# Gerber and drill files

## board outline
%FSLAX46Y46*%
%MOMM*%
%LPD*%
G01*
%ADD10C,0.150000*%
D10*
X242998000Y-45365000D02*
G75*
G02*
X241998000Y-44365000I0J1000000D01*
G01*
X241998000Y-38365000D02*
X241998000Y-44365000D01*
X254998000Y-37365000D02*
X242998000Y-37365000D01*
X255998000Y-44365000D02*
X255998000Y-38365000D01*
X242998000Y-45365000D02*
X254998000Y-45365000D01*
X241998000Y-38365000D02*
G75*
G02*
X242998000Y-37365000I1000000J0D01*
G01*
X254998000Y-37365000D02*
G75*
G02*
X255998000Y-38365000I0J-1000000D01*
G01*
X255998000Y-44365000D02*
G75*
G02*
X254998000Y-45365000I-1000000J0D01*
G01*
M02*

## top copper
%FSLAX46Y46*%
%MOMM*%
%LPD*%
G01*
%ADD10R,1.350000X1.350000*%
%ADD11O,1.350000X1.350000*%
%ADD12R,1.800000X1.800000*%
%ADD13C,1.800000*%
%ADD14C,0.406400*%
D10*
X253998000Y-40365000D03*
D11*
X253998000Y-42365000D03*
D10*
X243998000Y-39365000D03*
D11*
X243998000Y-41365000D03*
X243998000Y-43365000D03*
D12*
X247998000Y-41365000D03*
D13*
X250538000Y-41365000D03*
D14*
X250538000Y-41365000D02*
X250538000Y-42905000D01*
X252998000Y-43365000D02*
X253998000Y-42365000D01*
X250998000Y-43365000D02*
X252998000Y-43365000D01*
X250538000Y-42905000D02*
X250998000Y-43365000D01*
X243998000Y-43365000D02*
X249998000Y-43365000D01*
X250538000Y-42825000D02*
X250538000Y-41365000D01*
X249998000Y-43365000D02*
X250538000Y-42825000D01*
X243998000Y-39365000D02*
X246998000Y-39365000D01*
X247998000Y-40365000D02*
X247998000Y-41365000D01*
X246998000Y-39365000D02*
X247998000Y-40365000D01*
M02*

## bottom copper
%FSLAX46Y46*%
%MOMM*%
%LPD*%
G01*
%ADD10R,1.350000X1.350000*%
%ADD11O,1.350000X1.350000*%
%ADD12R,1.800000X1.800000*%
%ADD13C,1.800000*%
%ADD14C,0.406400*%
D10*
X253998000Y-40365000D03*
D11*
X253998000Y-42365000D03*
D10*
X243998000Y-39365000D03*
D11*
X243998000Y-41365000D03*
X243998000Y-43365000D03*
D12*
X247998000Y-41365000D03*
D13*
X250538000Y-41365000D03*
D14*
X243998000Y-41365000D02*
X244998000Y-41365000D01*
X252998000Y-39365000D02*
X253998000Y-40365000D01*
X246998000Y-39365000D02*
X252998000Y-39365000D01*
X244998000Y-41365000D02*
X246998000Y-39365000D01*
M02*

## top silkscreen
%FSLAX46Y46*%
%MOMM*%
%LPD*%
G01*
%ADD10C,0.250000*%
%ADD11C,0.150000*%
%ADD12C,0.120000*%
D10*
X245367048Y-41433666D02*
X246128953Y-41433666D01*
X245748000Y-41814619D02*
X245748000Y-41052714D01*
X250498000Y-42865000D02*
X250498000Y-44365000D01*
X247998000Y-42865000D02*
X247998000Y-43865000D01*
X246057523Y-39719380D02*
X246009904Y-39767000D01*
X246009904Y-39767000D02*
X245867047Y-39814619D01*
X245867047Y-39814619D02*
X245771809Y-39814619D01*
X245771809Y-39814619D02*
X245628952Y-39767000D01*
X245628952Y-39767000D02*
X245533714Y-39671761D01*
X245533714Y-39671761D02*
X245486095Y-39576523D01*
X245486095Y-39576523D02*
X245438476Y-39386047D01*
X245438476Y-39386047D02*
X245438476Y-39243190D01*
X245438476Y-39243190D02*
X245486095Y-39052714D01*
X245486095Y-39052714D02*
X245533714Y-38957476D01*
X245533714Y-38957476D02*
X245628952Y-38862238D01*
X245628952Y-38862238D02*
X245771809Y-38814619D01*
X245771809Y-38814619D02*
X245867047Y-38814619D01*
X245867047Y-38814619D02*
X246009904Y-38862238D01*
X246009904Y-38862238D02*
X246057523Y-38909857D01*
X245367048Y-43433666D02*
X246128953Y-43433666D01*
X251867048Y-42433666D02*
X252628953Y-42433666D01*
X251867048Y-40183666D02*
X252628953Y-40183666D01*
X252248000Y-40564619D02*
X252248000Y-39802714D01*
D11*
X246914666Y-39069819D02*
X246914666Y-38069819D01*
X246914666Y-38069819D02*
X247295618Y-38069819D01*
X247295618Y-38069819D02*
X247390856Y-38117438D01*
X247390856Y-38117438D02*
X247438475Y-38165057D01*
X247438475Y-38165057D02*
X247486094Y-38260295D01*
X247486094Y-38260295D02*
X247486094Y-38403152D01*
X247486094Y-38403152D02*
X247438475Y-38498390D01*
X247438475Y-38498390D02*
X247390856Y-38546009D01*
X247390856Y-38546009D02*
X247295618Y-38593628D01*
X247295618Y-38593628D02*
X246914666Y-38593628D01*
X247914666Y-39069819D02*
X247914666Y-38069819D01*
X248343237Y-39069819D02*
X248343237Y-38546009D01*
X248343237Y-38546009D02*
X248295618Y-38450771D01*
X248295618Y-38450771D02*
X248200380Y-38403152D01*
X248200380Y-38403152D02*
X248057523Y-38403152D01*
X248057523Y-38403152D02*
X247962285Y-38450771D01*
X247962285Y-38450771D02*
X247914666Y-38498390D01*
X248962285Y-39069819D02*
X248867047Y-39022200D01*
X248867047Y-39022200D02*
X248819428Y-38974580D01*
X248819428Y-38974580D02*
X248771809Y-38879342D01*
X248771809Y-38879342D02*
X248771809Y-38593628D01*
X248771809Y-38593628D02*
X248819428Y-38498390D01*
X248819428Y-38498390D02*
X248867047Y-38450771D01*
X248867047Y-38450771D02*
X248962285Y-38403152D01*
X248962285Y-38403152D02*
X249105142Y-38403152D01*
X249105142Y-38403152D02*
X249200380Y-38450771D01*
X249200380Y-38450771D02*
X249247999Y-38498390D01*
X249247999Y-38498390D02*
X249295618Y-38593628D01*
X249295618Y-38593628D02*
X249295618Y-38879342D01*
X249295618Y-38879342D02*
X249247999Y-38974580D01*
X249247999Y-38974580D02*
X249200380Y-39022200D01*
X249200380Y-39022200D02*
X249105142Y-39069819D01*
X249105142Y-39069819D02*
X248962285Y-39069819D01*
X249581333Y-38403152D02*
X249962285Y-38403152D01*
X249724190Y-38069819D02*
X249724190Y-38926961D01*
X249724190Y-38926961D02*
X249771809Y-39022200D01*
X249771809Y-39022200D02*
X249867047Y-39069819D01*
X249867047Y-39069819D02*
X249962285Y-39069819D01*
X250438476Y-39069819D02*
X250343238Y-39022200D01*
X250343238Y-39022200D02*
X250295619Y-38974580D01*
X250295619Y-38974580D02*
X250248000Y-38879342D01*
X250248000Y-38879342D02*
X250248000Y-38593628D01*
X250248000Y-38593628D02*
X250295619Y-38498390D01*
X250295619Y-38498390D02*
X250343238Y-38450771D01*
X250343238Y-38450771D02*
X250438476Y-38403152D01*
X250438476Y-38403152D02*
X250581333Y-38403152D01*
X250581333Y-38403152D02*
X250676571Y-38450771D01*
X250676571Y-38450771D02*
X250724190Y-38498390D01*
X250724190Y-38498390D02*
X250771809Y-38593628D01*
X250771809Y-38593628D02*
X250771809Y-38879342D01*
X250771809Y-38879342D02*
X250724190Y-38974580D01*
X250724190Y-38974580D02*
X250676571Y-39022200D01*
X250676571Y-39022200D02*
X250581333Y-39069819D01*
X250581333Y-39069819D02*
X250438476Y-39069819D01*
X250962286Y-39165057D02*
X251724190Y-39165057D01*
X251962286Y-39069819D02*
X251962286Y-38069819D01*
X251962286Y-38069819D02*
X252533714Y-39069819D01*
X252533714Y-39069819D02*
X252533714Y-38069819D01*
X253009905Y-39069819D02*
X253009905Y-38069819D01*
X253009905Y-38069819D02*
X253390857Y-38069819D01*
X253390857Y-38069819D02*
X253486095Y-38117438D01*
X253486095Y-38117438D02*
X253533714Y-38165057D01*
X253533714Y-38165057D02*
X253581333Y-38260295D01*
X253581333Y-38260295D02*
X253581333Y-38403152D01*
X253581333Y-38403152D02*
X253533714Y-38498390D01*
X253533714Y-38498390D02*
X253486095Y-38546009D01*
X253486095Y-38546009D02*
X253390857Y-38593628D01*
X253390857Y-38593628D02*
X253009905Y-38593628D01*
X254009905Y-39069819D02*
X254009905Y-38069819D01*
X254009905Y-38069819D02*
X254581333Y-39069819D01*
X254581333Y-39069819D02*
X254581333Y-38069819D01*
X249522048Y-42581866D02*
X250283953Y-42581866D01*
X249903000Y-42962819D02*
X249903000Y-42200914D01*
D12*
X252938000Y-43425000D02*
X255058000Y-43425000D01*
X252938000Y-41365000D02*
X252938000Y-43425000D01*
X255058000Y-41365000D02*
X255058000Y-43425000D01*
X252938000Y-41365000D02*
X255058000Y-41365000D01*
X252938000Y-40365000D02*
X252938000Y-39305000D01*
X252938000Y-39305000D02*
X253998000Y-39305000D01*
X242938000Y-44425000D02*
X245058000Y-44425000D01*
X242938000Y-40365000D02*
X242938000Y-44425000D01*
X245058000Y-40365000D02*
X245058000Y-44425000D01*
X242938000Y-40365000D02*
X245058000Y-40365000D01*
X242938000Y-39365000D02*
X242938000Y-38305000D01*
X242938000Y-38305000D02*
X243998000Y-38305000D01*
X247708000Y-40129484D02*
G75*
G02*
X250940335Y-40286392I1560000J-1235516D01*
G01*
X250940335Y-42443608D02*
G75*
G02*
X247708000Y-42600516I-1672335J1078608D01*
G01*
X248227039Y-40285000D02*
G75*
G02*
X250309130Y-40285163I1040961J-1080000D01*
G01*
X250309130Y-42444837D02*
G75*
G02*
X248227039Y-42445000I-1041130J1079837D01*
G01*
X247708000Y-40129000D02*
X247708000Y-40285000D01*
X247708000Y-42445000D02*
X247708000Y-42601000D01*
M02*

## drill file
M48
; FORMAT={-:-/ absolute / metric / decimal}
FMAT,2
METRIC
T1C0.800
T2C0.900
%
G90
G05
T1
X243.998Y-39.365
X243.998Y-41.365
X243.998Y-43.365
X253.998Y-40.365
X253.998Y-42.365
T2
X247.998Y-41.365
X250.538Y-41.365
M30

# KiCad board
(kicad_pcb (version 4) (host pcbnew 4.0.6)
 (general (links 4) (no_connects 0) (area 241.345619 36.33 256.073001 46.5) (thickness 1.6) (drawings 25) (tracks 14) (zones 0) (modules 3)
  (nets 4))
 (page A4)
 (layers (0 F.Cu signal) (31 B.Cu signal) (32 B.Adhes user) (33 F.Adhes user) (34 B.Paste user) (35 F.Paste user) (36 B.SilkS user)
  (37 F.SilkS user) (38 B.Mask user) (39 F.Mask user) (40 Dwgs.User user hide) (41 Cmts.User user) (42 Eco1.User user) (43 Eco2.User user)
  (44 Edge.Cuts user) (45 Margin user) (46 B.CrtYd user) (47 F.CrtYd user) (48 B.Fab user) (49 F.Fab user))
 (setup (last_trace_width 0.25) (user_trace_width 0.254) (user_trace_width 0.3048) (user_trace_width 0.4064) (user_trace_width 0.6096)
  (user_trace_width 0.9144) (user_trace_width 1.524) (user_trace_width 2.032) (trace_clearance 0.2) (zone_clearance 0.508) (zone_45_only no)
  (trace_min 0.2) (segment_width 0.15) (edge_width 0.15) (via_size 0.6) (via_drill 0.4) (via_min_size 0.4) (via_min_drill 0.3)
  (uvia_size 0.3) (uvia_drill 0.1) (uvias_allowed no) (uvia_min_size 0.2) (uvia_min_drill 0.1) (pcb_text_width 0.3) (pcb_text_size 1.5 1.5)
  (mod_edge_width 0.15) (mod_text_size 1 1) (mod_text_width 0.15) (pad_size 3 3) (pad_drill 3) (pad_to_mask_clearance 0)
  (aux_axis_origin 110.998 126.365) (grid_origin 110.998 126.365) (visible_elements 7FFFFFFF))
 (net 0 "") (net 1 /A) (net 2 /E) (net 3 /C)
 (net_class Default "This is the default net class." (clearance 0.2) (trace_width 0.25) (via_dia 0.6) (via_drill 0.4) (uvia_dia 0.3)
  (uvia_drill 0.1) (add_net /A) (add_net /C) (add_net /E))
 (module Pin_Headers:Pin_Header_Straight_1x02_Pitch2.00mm (layer F.Cu) (at 253.998 40.365)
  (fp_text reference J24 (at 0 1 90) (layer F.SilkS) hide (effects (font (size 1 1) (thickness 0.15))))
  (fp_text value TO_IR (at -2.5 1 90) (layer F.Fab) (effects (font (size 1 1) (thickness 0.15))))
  (fp_line (start -1.06 3.06) (end 1.06 3.06) (layer F.SilkS) (width 0.12))
  (fp_line (start -1.06 1) (end -1.06 3.06) (layer F.SilkS) (width 0.12))
  (fp_line (start 1.06 1) (end 1.06 3.06) (layer F.SilkS) (width 0.12))
  (fp_line (start -1.06 1) (end 1.06 1) (layer F.SilkS) (width 0.12))
  (fp_line (start -1.06 0) (end -1.06 -1.06) (layer F.SilkS) (width 0.12))
  (fp_line (start -1.06 -1.06) (end 0 -1.06) (layer F.SilkS) (width 0.12))
  (pad 1 thru_hole rect (at 0 0) (size 1.35 1.35) (drill 0.8) (layers *.Cu *.Mask) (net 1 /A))
  (pad 2 thru_hole oval (at 0 2) (size 1.35 1.35) (drill 0.8) (layers *.Cu *.Mask) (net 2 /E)))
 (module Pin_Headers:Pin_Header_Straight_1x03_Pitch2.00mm (layer F.Cu) (at 243.998 39.365)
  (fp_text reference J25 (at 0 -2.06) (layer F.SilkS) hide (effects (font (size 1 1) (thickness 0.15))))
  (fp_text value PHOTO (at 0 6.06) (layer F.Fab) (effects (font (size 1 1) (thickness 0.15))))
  (fp_line (start -1.06 5.06) (end 1.06 5.06) (layer F.SilkS) (width 0.12))
  (fp_line (start -1.06 1) (end -1.06 5.06) (layer F.SilkS) (width 0.12))
  (fp_line (start 1.06 1) (end 1.06 5.06) (layer F.SilkS) (width 0.12))
  (fp_line (start -1.06 1) (end 1.06 1) (layer F.SilkS) (width 0.12))
  (fp_line (start -1.06 0) (end -1.06 -1.06) (layer F.SilkS) (width 0.12))
  (fp_line (start -1.06 -1.06) (end 0 -1.06) (layer F.SilkS) (width 0.12))
  (pad 1 thru_hole rect (at 0 0) (size 1.35 1.35) (drill 0.8) (layers *.Cu *.Mask) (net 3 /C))
  (pad 2 thru_hole oval (at 0 2) (size 1.35 1.35) (drill 0.8) (layers *.Cu *.Mask) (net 1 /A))
  (pad 3 thru_hole oval (at 0 4) (size 1.35 1.35) (drill 0.8) (layers *.Cu *.Mask) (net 2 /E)))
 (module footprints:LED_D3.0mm (layer F.Cu) (at 247.998 41.365)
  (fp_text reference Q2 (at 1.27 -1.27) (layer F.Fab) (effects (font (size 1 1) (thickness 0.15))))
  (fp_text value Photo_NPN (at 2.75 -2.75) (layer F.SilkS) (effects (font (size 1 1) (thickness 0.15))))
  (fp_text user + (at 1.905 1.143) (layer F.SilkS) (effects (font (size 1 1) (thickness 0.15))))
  (fp_arc (start 1.27 0) (end -0.29 -1.235516) (angle 108.8) (layer F.SilkS) (width 0.12))
  (fp_arc (start 1.27 0) (end -0.29 1.235516) (angle -108.8) (layer F.SilkS) (width 0.12))
  (fp_arc (start 1.27 0) (end 0.229039 -1.08) (angle 87.9) (layer F.SilkS) (width 0.12))
  (fp_arc (start 1.27 0) (end 0.229039 1.08) (angle -87.9) (layer F.SilkS) (width 0.12))
  (fp_line (start -0.29 -1.236) (end -0.29 -1.08) (layer F.SilkS) (width 0.12))
  (fp_line (start -0.29 1.08) (end -0.29 1.236) (layer F.SilkS) (width 0.12))
  (pad 1 thru_hole rect (at 0 0) (size 1.8 1.8) (drill 0.9) (layers *.Cu *.Mask) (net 3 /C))
  (pad 2 thru_hole circle (at 2.54 0) (size 1.8 1.8) (drill 0.9) (layers *.Cu *.Mask) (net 2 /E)))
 (gr_arc (start 242.998 44.365) (end 242.998 45.365) (angle 90) (layer Edge.Cuts) (width 0.15))
 (gr_line (start 241.998 38.365) (end 241.998 44.365) (angle 90) (layer Edge.Cuts) (width 0.15))
 (gr_line (start 254.998 37.365) (end 242.998 37.365) (angle 90) (layer Edge.Cuts) (width 0.15))
 (gr_line (start 255.998 44.365) (end 255.998 38.365) (angle 90) (layer Edge.Cuts) (width 0.15))
 (gr_line (start 242.998 45.365) (end 254.998 45.365) (angle 90) (layer Edge.Cuts) (width 0.15))
 (gr_arc (start 242.998 38.365) (end 241.998 38.365) (angle 90) (layer Edge.Cuts) (width 0.15))
 (gr_arc (start 254.998 38.365) (end 254.998 37.365) (angle 90) (layer Edge.Cuts) (width 0.15))
 (gr_arc (start 254.998 44.365) (end 255.998 44.365) (angle 90) (layer Edge.Cuts) (width 0.15))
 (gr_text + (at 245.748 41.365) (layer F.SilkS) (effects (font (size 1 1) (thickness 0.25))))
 (gr_line (start 250.498 42.865) (end 250.498 44.365) (angle 90) (layer F.SilkS) (width 0.25))
 (gr_line (start 247.998 42.865) (end 247.998 43.865) (angle 90) (layer F.SilkS) (width 0.25))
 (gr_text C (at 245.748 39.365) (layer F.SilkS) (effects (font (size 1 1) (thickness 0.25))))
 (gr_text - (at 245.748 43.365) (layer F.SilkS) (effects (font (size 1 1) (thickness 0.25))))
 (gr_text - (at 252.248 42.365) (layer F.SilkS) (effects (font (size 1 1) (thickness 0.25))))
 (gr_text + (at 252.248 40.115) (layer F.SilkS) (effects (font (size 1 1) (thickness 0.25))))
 (segment (start 243.998 41.365) (end 244.998 41.365) (width 0.4064) (layer B.Cu) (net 1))
 (segment (start 252.998 39.365) (end 253.998 40.365) (width 0.4064) (layer B.Cu) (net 1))
 (segment (start 246.998 39.365) (end 252.998 39.365) (width 0.4064) (layer B.Cu) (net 1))
 (segment (start 244.998 41.365) (end 246.998 39.365) (width 0.4064) (layer B.Cu) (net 1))
 (segment (start 250.538 41.365) (end 250.538 42.905) (width 0.4064) (layer F.Cu) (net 2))
 (segment (start 252.998 43.365) (end 253.998 42.365) (width 0.4064) (layer F.Cu) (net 2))
 (segment (start 250.998 43.365) (end 252.998 43.365) (width 0.4064) (layer F.Cu) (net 2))
 (segment (start 250.538 42.905) (end 250.998 43.365) (width 0.4064) (layer F.Cu) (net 2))
 (segment (start 243.998 43.365) (end 249.998 43.365) (width 0.4064) (layer F.Cu) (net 2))
 (segment (start 250.538 42.825) (end 250.538 41.365) (width 0.4064) (layer F.Cu) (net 2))
 (segment (start 249.998 43.365) (end 250.538 42.825) (width 0.4064) (layer F.Cu) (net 2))
 (segment (start 243.998 39.365) (end 246.998 39.365) (width 0.4064) (layer F.Cu) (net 3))
 (segment (start 247.998 40.365) (end 247.998 41.365) (width 0.4064) (layer F.Cu) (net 3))
 (segment (start 246.998 39.365) (end 247.998 40.365) (width 0.4064) (layer F.Cu) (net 3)))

